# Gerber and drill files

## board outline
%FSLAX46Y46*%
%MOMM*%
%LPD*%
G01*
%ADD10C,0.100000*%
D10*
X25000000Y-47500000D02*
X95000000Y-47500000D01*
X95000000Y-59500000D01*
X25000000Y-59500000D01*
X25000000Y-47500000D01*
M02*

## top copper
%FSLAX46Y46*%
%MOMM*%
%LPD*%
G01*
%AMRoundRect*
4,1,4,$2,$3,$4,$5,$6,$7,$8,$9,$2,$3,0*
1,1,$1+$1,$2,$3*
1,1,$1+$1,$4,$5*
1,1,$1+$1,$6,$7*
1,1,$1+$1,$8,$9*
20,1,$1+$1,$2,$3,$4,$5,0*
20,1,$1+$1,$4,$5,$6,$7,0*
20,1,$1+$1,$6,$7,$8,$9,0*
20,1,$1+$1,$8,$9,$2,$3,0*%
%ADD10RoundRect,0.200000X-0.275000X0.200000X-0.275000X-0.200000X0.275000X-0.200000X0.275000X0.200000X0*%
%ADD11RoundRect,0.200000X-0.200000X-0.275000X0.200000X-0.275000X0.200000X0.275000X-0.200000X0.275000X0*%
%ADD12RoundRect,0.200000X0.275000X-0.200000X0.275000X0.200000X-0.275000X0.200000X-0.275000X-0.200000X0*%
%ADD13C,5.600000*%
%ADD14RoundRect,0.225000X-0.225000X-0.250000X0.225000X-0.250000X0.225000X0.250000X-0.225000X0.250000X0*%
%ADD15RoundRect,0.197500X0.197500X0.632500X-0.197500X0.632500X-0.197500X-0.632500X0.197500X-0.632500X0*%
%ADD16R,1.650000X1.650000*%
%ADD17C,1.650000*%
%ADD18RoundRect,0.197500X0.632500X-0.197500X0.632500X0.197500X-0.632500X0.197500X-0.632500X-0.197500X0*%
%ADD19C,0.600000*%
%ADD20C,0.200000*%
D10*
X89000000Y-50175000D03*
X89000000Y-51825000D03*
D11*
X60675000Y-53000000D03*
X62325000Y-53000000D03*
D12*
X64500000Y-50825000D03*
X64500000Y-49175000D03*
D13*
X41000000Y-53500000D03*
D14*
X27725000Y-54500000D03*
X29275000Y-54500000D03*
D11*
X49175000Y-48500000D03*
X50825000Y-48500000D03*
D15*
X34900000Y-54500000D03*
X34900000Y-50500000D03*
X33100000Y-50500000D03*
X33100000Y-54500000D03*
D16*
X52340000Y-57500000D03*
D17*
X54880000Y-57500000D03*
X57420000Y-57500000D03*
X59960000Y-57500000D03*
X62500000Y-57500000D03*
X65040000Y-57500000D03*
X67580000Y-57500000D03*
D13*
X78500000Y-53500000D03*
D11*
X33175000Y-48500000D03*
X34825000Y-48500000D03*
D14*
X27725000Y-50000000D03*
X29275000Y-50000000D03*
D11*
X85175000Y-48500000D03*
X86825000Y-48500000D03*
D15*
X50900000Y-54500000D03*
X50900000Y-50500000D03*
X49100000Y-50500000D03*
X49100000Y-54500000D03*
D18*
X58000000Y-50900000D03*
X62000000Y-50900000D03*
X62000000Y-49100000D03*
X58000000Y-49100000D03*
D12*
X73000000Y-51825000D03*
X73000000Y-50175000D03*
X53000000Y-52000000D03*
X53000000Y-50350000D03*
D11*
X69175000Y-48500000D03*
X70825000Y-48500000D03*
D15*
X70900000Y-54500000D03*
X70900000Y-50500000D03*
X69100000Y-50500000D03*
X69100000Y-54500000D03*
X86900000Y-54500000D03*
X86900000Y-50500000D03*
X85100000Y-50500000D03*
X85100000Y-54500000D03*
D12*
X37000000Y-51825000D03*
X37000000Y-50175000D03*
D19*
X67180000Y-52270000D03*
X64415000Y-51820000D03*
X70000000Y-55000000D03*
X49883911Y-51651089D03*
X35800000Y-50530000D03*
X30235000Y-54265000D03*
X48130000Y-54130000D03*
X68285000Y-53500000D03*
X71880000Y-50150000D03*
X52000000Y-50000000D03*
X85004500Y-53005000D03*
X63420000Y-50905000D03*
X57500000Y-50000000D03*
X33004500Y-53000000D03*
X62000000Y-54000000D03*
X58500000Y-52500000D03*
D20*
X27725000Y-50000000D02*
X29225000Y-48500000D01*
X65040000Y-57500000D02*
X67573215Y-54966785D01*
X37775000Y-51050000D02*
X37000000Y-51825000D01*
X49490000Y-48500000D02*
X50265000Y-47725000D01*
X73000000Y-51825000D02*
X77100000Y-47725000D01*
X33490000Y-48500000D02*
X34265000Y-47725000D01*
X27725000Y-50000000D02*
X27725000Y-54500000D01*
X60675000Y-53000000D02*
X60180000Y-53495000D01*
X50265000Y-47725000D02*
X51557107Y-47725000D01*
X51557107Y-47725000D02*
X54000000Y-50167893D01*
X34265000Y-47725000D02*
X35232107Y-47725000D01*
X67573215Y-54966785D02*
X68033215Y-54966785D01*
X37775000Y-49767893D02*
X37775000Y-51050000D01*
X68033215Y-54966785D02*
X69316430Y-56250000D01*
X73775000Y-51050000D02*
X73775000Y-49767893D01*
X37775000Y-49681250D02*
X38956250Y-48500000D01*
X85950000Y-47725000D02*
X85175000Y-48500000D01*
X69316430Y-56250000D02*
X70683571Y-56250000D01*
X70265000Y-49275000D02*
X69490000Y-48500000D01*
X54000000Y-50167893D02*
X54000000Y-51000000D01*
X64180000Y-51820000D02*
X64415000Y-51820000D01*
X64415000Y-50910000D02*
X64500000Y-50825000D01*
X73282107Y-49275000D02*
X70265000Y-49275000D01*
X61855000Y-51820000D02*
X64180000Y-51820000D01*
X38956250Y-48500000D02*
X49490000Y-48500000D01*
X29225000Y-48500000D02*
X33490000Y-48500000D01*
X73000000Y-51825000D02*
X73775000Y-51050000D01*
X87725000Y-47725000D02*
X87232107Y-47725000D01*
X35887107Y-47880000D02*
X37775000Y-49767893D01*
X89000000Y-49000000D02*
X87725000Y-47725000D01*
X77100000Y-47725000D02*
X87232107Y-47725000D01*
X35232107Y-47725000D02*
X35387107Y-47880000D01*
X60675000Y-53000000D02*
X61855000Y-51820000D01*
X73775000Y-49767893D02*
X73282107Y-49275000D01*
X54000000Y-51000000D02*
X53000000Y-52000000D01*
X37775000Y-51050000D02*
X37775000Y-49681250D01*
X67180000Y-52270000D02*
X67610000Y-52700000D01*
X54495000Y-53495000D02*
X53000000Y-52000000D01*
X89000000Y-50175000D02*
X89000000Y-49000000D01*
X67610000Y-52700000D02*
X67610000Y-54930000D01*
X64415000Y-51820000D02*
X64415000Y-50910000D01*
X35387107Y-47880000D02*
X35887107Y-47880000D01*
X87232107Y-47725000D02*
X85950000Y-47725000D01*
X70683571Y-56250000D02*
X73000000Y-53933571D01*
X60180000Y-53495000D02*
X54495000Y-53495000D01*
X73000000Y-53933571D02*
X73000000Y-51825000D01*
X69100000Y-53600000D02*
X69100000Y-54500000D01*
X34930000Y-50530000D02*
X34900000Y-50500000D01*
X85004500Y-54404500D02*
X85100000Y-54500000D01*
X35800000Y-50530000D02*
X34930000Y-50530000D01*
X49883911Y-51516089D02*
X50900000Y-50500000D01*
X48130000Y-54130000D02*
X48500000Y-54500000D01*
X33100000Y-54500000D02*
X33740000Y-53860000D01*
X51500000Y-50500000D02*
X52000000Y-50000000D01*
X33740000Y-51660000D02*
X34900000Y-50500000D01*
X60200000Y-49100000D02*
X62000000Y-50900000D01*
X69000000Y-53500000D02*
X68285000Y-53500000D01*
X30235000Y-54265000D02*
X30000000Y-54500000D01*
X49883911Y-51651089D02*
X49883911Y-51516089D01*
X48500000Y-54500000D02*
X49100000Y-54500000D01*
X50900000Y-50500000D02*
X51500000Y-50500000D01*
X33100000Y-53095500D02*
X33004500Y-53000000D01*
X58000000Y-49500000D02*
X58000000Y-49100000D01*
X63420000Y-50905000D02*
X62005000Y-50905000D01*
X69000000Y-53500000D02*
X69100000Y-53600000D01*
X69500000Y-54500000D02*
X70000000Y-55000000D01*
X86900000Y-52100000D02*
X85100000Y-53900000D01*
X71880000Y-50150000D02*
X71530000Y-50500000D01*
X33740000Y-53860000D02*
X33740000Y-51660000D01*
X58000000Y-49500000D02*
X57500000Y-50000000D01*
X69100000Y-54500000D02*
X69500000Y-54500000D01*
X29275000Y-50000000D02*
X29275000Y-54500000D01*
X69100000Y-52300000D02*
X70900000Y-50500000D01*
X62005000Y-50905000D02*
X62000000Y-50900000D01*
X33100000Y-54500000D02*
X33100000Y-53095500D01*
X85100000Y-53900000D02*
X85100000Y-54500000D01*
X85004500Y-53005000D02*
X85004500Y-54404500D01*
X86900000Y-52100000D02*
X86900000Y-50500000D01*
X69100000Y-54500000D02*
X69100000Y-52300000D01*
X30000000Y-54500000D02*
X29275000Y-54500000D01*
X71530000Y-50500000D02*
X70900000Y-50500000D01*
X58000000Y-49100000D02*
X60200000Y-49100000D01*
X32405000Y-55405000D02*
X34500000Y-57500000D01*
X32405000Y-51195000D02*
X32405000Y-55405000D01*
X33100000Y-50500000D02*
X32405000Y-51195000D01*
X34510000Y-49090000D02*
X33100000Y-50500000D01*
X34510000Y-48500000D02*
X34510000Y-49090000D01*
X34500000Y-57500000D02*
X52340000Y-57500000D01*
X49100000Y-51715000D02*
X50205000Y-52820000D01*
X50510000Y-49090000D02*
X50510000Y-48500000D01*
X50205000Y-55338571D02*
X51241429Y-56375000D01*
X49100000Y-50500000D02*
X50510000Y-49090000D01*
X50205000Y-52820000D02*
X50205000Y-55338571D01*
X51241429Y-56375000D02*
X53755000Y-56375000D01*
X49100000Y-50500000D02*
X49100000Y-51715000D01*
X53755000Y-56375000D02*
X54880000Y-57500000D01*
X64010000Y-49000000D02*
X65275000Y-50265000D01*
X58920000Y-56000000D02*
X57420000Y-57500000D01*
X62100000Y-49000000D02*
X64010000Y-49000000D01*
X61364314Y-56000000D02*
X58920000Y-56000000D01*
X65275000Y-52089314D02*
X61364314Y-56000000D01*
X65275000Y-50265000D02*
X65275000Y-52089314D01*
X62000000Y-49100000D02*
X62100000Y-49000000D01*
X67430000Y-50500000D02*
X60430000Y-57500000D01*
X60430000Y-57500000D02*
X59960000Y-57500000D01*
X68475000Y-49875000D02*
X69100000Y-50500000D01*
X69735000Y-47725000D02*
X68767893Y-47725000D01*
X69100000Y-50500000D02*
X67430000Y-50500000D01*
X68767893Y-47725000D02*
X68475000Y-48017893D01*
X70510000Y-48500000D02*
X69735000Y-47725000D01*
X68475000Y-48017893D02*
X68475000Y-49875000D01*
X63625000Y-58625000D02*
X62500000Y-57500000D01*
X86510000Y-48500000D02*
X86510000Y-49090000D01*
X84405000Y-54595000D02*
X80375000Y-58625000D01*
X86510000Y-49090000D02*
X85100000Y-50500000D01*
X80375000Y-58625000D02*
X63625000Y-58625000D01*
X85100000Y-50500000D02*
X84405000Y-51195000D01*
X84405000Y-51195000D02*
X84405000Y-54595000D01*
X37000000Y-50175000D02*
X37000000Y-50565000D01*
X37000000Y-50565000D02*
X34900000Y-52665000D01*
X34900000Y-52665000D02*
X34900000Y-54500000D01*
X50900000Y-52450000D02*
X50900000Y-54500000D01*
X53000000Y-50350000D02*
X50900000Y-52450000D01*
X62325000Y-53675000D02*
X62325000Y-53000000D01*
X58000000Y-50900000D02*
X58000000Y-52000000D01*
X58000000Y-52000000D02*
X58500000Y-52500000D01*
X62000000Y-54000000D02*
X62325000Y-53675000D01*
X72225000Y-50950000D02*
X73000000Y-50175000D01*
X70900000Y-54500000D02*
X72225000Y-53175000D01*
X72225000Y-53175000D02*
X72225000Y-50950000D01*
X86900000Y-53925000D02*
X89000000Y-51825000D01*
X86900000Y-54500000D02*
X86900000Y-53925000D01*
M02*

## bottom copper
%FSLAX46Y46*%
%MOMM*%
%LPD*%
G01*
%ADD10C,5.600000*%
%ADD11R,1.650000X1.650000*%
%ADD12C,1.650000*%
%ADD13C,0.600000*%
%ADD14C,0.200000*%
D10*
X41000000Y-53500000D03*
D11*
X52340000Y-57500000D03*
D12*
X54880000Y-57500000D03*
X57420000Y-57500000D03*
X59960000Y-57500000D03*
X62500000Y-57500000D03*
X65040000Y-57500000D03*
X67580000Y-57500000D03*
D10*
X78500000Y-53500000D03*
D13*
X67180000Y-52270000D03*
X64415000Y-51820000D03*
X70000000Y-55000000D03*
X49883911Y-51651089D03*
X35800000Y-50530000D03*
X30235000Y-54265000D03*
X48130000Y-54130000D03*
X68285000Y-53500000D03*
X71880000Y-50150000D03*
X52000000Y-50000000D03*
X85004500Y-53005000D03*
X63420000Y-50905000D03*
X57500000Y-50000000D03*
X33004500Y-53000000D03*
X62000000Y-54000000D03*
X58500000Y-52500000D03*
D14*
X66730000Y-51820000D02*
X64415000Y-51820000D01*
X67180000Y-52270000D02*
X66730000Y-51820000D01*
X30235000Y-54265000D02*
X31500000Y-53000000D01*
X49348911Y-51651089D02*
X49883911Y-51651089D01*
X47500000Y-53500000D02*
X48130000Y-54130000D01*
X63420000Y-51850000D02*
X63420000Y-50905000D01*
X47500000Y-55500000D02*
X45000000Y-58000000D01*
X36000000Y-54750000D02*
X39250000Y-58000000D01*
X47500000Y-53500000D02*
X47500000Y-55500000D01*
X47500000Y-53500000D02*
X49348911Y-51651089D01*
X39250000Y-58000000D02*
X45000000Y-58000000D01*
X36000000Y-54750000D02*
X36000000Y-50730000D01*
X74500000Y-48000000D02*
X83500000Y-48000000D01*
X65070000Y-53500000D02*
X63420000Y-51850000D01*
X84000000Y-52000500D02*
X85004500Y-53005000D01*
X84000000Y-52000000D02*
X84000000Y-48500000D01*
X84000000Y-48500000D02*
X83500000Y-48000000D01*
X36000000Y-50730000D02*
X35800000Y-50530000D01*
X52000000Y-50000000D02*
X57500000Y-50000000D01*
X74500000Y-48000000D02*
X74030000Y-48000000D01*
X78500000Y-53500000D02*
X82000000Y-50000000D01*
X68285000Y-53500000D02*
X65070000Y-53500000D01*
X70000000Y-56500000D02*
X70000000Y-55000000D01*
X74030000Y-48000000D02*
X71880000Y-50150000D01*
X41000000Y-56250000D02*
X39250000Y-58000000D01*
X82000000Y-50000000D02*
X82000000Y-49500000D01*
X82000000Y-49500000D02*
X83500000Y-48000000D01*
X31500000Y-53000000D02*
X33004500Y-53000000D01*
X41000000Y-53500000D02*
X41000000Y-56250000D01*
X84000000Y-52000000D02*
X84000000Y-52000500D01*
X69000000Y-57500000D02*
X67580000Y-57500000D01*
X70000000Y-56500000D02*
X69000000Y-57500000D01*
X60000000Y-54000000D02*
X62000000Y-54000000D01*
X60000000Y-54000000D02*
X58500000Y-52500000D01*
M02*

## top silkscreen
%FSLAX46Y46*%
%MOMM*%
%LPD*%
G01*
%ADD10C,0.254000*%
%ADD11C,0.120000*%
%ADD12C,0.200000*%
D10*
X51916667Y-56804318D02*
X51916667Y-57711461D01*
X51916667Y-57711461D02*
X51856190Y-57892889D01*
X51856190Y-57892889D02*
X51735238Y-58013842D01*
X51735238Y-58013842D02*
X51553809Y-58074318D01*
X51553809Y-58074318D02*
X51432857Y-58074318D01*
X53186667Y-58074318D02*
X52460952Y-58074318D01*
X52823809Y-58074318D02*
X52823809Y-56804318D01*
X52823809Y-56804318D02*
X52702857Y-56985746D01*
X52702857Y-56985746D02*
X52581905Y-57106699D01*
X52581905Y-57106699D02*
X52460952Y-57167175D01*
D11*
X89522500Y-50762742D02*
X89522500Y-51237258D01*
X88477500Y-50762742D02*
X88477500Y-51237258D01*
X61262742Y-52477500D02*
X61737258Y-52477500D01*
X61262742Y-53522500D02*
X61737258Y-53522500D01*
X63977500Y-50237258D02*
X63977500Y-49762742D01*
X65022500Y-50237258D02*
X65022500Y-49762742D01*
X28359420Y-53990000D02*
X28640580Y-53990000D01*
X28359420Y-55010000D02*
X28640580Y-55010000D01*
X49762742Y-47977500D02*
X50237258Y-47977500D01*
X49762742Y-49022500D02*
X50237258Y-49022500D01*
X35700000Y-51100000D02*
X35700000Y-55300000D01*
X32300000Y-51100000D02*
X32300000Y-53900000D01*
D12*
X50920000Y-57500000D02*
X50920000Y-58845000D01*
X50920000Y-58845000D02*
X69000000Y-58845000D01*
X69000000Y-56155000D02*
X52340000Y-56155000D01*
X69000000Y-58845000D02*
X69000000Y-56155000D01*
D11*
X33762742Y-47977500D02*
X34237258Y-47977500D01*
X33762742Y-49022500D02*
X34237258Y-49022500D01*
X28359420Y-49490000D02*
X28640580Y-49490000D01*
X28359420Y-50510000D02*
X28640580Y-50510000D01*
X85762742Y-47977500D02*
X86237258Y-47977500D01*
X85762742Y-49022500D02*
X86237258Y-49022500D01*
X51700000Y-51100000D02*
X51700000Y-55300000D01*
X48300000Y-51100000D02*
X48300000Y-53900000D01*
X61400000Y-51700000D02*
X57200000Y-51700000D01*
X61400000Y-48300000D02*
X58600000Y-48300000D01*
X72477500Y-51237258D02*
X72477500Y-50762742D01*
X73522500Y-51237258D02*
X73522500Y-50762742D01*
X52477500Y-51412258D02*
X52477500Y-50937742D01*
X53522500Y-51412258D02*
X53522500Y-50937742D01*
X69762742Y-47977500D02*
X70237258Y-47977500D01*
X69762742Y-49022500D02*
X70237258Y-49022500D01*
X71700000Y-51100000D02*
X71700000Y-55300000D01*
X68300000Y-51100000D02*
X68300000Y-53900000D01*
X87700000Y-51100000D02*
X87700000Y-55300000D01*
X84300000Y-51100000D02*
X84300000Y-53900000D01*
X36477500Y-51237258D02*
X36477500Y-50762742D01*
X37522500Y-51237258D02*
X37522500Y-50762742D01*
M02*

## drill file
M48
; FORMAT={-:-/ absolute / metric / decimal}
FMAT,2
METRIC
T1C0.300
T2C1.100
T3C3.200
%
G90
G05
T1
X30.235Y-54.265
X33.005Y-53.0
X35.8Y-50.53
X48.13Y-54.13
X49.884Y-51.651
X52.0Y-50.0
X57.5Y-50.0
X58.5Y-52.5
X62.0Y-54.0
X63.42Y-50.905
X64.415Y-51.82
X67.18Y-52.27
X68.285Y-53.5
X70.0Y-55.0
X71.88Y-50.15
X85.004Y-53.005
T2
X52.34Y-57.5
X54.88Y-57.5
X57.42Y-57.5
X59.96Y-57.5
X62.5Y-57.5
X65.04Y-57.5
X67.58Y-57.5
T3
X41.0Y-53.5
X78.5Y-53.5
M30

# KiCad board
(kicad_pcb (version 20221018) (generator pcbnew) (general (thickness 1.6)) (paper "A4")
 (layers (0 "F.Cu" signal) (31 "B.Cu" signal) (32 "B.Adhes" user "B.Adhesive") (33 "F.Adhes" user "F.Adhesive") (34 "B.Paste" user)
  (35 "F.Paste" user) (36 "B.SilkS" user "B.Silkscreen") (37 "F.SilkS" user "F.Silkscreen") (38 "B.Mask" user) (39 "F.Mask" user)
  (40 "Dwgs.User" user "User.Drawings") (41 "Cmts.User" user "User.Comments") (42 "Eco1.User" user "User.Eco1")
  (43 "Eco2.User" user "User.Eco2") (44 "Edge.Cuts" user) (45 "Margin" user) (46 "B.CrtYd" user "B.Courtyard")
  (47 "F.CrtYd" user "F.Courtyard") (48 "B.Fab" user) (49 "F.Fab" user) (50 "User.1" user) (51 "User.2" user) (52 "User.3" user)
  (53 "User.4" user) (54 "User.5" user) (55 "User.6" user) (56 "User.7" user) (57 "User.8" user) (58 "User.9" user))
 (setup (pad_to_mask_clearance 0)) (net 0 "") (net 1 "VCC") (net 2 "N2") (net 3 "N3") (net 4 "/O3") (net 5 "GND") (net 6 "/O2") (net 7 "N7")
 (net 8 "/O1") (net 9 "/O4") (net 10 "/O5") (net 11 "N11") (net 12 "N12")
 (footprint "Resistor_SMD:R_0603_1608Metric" (layer "F.Cu") (at 89 51 -90)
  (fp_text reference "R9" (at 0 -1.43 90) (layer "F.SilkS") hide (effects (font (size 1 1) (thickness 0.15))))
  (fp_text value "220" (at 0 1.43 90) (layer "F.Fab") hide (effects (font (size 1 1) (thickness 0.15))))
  (fp_line (start -0.237258 -0.5225) (end 0.237258 -0.5225) (stroke (width 0.12) (type solid)) (layer "F.SilkS"))
  (fp_line (start -0.237258 0.5225) (end 0.237258 0.5225) (stroke (width 0.12) (type solid)) (layer "F.SilkS"))
  (pad "1" smd roundrect (at -0.825 0 270) (size 0.8 0.95) (layers "F.Cu" "F.Paste" "F.Mask") (roundrect_rratio 0.25) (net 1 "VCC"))
  (pad "2" smd roundrect (at 0.825 0 270) (size 0.8 0.95) (layers "F.Cu" "F.Paste" "F.Mask") (roundrect_rratio 0.25) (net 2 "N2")))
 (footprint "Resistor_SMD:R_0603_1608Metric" (layer "F.Cu") (at 61.5 53)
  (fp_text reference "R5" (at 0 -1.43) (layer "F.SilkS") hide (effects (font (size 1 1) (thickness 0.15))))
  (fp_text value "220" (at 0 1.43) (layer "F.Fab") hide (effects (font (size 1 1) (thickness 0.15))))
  (fp_line (start -0.237258 -0.5225) (end 0.237258 -0.5225) (stroke (width 0.12) (type solid)) (layer "F.SilkS"))
  (fp_line (start -0.237258 0.5225) (end 0.237258 0.5225) (stroke (width 0.12) (type solid)) (layer "F.SilkS"))
  (pad "1" smd roundrect (at -0.825 0) (size 0.8 0.95) (layers "F.Cu" "F.Paste" "F.Mask") (roundrect_rratio 0.25) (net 1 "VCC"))
  (pad "2" smd roundrect (at 0.825 0) (size 0.8 0.95) (layers "F.Cu" "F.Paste" "F.Mask") (roundrect_rratio 0.25) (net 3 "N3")))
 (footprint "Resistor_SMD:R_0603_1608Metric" (layer "F.Cu") (at 64.5 50 90)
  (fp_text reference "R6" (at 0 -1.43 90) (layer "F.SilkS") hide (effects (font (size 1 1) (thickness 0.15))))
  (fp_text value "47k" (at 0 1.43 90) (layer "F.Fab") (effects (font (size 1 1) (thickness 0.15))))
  (fp_line (start -0.237258 -0.5225) (end 0.237258 -0.5225) (stroke (width 0.12) (type solid)) (layer "F.SilkS"))
  (fp_line (start -0.237258 0.5225) (end 0.237258 0.5225) (stroke (width 0.12) (type solid)) (layer "F.SilkS"))
  (pad "1" smd roundrect (at -0.825 0 90) (size 0.8 0.95) (layers "F.Cu" "F.Paste" "F.Mask") (roundrect_rratio 0.25) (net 1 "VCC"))
  (pad "2" smd roundrect (at 0.825 0 90) (size 0.8 0.95) (layers "F.Cu" "F.Paste" "F.Mask") (roundrect_rratio 0.25) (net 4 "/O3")))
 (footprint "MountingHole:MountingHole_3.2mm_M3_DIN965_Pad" (layer "F.Cu") (at 41 53.5)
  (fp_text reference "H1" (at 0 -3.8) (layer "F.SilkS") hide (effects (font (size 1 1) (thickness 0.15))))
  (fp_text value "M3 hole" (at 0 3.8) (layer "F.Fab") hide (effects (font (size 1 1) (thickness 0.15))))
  (pad "1" thru_hole circle (at 0 0) (size 5.6 5.6) (drill 3.2) (layers "*.Cu" "*.Mask") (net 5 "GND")))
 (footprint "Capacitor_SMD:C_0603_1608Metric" (layer "F.Cu") (at 28.5 54.5)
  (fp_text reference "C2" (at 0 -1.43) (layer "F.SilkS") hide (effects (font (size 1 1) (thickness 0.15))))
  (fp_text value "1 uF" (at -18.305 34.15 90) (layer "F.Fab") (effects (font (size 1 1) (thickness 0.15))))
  (fp_line (start -0.14058 -0.51) (end 0.14058 -0.51) (stroke (width 0.12) (type solid)) (layer "F.SilkS"))
  (fp_line (start -0.14058 0.51) (end 0.14058 0.51) (stroke (width 0.12) (type solid)) (layer "F.SilkS"))
  (pad "1" smd roundrect (at -0.775 0) (size 0.9 0.95) (layers "F.Cu" "F.Paste" "F.Mask") (roundrect_rratio 0.25) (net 1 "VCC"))
  (pad "2" smd roundrect (at 0.775 0) (size 0.9 0.95) (layers "F.Cu" "F.Paste" "F.Mask") (roundrect_rratio 0.25) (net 5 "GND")))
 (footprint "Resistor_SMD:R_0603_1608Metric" (layer "F.Cu") (at 50 48.5)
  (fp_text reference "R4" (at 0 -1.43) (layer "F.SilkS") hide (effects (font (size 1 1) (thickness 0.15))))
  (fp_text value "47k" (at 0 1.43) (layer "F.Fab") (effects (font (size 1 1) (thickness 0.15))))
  (fp_line (start -0.237258 -0.5225) (end 0.237258 -0.5225) (stroke (width 0.12) (type solid)) (layer "F.SilkS"))
  (fp_line (start -0.237258 0.5225) (end 0.237258 0.5225) (stroke (width 0.12) (type solid)) (layer "F.SilkS"))
  (pad "1" smd roundrect (at -0.825 0) (size 0.8 0.95) (layers "F.Cu" "F.Paste" "F.Mask") (roundrect_rratio 0.25) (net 1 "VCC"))
  (pad "2" smd roundrect (at 0.825 0) (size 0.8 0.95) (layers "F.Cu" "F.Paste" "F.Mask") (roundrect_rratio 0.25) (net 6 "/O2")))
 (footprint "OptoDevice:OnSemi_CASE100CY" (layer "F.Cu") (at 34 52.5 180)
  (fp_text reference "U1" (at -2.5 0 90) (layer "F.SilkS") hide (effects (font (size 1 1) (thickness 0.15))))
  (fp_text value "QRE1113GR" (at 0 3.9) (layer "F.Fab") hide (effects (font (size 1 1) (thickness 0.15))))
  (fp_line (start -1.7 1.4) (end -1.7 -2.8) (stroke (width 0.12) (type solid)) (layer "F.SilkS"))
  (fp_line (start 1.7 1.4) (end 1.7 -1.4) (stroke (width 0.12) (type solid)) (layer "F.SilkS"))
  (pad "1" smd roundrect (at -0.9 -2 180) (size 0.79 1.66) (layers "F.Cu" "F.Paste" "F.Mask") (roundrect_rratio 0.25) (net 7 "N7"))
  (pad "2" smd roundrect (at -0.9 2 180) (size 0.79 1.66) (layers "F.Cu" "F.Paste" "F.Mask") (roundrect_rratio 0.25) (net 5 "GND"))
  (pad "3" smd roundrect (at 0.9 2 180) (size 0.79 1.66) (layers "F.Cu" "F.Paste" "F.Mask") (roundrect_rratio 0.25) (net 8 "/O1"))
  (pad "4" smd roundrect (at 0.9 -2 180) (size 0.79 1.66) (layers "F.Cu" "F.Paste" "F.Mask") (roundrect_rratio 0.25) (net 5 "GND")))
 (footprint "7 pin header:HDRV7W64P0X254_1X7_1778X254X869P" (layer "F.Cu") (at 52.34 57.5)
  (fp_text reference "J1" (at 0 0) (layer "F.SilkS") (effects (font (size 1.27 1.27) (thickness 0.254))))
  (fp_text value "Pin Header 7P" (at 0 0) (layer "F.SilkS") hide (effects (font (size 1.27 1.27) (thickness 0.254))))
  (fp_line (start -1.42 0) (end -1.42 1.345) (stroke (width 0.2) (type solid)) (layer "F.SilkS"))
  (fp_line (start -1.42 1.345) (end 16.66 1.345) (stroke (width 0.2) (type solid)) (layer "F.SilkS"))
  (fp_line (start 16.66 -1.345) (end 0 -1.345) (stroke (width 0.2) (type solid)) (layer "F.SilkS"))
  (fp_line (start 16.66 1.345) (end 16.66 -1.345) (stroke (width 0.2) (type solid)) (layer "F.SilkS"))
  (pad "1" thru_hole rect (at 0 0) (size 1.65 1.65) (drill 1.1) (layers "*.Cu" "*.Mask") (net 8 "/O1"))
  (pad "2" thru_hole circle (at 2.54 0) (size 1.65 1.65) (drill 1.1) (layers "*.Cu" "*.Mask") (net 6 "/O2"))
  (pad "3" thru_hole circle (at 5.08 0) (size 1.65 1.65) (drill 1.1) (layers "*.Cu" "*.Mask") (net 4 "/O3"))
  (pad "4" thru_hole circle (at 7.62 0) (size 1.65 1.65) (drill 1.1) (layers "*.Cu" "*.Mask") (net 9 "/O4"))
  (pad "5" thru_hole circle (at 10.16 0) (size 1.65 1.65) (drill 1.1) (layers "*.Cu" "*.Mask") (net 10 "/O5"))
  (pad "6" thru_hole circle (at 12.7 0) (size 1.65 1.65) (drill 1.1) (layers "*.Cu" "*.Mask") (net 1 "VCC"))
  (pad "7" thru_hole circle (at 15.24 0) (size 1.65 1.65) (drill 1.1) (layers "*.Cu" "*.Mask") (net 5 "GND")))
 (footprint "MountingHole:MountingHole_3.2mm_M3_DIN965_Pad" (layer "F.Cu") (at 78.5 53.5)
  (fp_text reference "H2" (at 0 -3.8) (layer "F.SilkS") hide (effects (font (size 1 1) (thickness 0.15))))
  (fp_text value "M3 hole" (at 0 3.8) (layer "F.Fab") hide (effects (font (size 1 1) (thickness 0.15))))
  (pad "1" thru_hole circle (at 0 0) (size 5.6 5.6) (drill 3.2) (layers "*.Cu" "*.Mask") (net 5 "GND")))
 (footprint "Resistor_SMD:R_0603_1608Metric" (layer "F.Cu") (at 34 48.5)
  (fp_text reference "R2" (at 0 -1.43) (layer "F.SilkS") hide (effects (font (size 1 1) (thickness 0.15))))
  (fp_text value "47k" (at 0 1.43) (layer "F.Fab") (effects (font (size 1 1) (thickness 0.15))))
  (fp_line (start -0.237258 -0.5225) (end 0.237258 -0.5225) (stroke (width 0.12) (type solid)) (layer "F.SilkS"))
  (fp_line (start -0.237258 0.5225) (end 0.237258 0.5225) (stroke (width 0.12) (type solid)) (layer "F.SilkS"))
  (pad "1" smd roundrect (at -0.825 0) (size 0.8 0.95) (layers "F.Cu" "F.Paste" "F.Mask") (roundrect_rratio 0.25) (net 1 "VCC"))
  (pad "2" smd roundrect (at 0.825 0) (size 0.8 0.95) (layers "F.Cu" "F.Paste" "F.Mask") (roundrect_rratio 0.25) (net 8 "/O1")))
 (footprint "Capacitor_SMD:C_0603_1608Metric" (layer "F.Cu") (at 28.5 50)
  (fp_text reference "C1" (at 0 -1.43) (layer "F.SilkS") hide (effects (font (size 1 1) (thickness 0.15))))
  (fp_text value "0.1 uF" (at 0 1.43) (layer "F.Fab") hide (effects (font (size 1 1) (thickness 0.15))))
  (fp_line (start -0.14058 -0.51) (end 0.14058 -0.51) (stroke (width 0.12) (type solid)) (layer "F.SilkS"))
  (fp_line (start -0.14058 0.51) (end 0.14058 0.51) (stroke (width 0.12) (type solid)) (layer "F.SilkS"))
  (pad "1" smd roundrect (at -0.775 0) (size 0.9 0.95) (layers "F.Cu" "F.Paste" "F.Mask") (roundrect_rratio 0.25) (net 1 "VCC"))
  (pad "2" smd roundrect (at 0.775 0) (size 0.9 0.95) (layers "F.Cu" "F.Paste" "F.Mask") (roundrect_rratio 0.25) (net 5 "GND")))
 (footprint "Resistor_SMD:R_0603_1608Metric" (layer "F.Cu") (at 86 48.5)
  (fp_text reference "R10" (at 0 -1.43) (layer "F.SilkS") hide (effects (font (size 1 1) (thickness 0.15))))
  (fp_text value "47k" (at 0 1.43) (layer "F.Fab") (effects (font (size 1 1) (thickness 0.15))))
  (fp_line (start -0.237258 -0.5225) (end 0.237258 -0.5225) (stroke (width 0.12) (type solid)) (layer "F.SilkS"))
  (fp_line (start -0.237258 0.5225) (end 0.237258 0.5225) (stroke (width 0.12) (type solid)) (layer "F.SilkS"))
  (pad "1" smd roundrect (at -0.825 0) (size 0.8 0.95) (layers "F.Cu" "F.Paste" "F.Mask") (roundrect_rratio 0.25) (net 1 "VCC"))
  (pad "2" smd roundrect (at 0.825 0) (size 0.8 0.95) (layers "F.Cu" "F.Paste" "F.Mask") (roundrect_rratio 0.25) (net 10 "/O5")))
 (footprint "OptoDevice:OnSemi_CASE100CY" (layer "F.Cu") (at 50 52.5 180)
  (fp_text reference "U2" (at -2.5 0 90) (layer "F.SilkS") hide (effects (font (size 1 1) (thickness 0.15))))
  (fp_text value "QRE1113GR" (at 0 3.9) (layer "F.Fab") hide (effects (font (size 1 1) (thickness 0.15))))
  (fp_line (start -1.7 1.4) (end -1.7 -2.8) (stroke (width 0.12) (type solid)) (layer "F.SilkS"))
  (fp_line (start 1.7 1.4) (end 1.7 -1.4) (stroke (width 0.12) (type solid)) (layer "F.SilkS"))
  (pad "1" smd roundrect (at -0.9 -2 180) (size 0.79 1.66) (layers "F.Cu" "F.Paste" "F.Mask") (roundrect_rratio 0.25) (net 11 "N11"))
  (pad "2" smd roundrect (at -0.9 2 180) (size 0.79 1.66) (layers "F.Cu" "F.Paste" "F.Mask") (roundrect_rratio 0.25) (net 5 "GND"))
  (pad "3" smd roundrect (at 0.9 2 180) (size 0.79 1.66) (layers "F.Cu" "F.Paste" "F.Mask") (roundrect_rratio 0.25) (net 6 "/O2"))
  (pad "4" smd roundrect (at 0.9 -2 180) (size 0.79 1.66) (layers "F.Cu" "F.Paste" "F.Mask") (roundrect_rratio 0.25) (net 5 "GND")))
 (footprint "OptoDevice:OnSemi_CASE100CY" (layer "F.Cu") (at 60 50 90)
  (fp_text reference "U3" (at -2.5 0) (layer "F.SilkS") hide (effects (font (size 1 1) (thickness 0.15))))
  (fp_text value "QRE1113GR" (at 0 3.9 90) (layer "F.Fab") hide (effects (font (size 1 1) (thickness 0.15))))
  (fp_line (start -1.7 1.4) (end -1.7 -2.8) (stroke (width 0.12) (type solid)) (layer "F.SilkS"))
  (fp_line (start 1.7 1.4) (end 1.7 -1.4) (stroke (width 0.12) (type solid)) (layer "F.SilkS"))
  (pad "1" smd roundrect (at -0.9 -2 90) (size 0.79 1.66) (layers "F.Cu" "F.Paste" "F.Mask") (roundrect_rratio 0.25) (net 3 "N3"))
  (pad "2" smd roundrect (at -0.9 2 90) (size 0.79 1.66) (layers "F.Cu" "F.Paste" "F.Mask") (roundrect_rratio 0.25) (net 5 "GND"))
  (pad "3" smd roundrect (at 0.9 2 90) (size 0.79 1.66) (layers "F.Cu" "F.Paste" "F.Mask") (roundrect_rratio 0.25) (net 4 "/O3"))
  (pad "4" smd roundrect (at 0.9 -2 90) (size 0.79 1.66) (layers "F.Cu" "F.Paste" "F.Mask") (roundrect_rratio 0.25) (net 5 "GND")))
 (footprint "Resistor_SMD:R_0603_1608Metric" (layer "F.Cu") (at 73 51 90)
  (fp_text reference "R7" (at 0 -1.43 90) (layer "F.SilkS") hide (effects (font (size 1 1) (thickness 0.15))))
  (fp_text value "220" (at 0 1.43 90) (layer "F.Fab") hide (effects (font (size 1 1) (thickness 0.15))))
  (fp_line (start -0.237258 -0.5225) (end 0.237258 -0.5225) (stroke (width 0.12) (type solid)) (layer "F.SilkS"))
  (fp_line (start -0.237258 0.5225) (end 0.237258 0.5225) (stroke (width 0.12) (type solid)) (layer "F.SilkS"))
  (pad "1" smd roundrect (at -0.825 0 90) (size 0.8 0.95) (layers "F.Cu" "F.Paste" "F.Mask") (roundrect_rratio 0.25) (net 1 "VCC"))
  (pad "2" smd roundrect (at 0.825 0 90) (size 0.8 0.95) (layers "F.Cu" "F.Paste" "F.Mask") (roundrect_rratio 0.25) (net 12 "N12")))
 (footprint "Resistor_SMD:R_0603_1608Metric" (layer "F.Cu") (at 53 51.175 90)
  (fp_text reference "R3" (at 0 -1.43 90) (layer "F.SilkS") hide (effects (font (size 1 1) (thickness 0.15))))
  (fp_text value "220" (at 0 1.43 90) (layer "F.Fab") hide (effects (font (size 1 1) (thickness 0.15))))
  (fp_line (start -0.237258 -0.5225) (end 0.237258 -0.5225) (stroke (width 0.12) (type solid)) (layer "F.SilkS"))
  (fp_line (start -0.237258 0.5225) (end 0.237258 0.5225) (stroke (width 0.12) (type solid)) (layer "F.SilkS"))
  (pad "1" smd roundrect (at -0.825 0 90) (size 0.8 0.95) (layers "F.Cu" "F.Paste" "F.Mask") (roundrect_rratio 0.25) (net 1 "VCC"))
  (pad "2" smd roundrect (at 0.825 0 90) (size 0.8 0.95) (layers "F.Cu" "F.Paste" "F.Mask") (roundrect_rratio 0.25) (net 11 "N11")))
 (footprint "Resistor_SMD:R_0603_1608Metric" (layer "F.Cu") (at 70 48.5)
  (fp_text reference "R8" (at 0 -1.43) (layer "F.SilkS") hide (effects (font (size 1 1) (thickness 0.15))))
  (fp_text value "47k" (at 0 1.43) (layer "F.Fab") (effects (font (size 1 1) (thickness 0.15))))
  (fp_line (start -0.237258 -0.5225) (end 0.237258 -0.5225) (stroke (width 0.12) (type solid)) (layer "F.SilkS"))
  (fp_line (start -0.237258 0.5225) (end 0.237258 0.5225) (stroke (width 0.12) (type solid)) (layer "F.SilkS"))
  (pad "1" smd roundrect (at -0.825 0) (size 0.8 0.95) (layers "F.Cu" "F.Paste" "F.Mask") (roundrect_rratio 0.25) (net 1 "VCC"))
  (pad "2" smd roundrect (at 0.825 0) (size 0.8 0.95) (layers "F.Cu" "F.Paste" "F.Mask") (roundrect_rratio 0.25) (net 9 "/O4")))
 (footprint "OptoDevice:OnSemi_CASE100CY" (layer "F.Cu") (at 70 52.5 180)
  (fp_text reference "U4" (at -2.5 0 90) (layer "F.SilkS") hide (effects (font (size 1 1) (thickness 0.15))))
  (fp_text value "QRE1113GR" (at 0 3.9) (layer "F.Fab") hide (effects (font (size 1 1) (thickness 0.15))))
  (fp_line (start -1.7 1.4) (end -1.7 -2.8) (stroke (width 0.12) (type solid)) (layer "F.SilkS"))
  (fp_line (start 1.7 1.4) (end 1.7 -1.4) (stroke (width 0.12) (type solid)) (layer "F.SilkS"))
  (pad "1" smd roundrect (at -0.9 -2 180) (size 0.79 1.66) (layers "F.Cu" "F.Paste" "F.Mask") (roundrect_rratio 0.25) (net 12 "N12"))
  (pad "2" smd roundrect (at -0.9 2 180) (size 0.79 1.66) (layers "F.Cu" "F.Paste" "F.Mask") (roundrect_rratio 0.25) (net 5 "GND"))
  (pad "3" smd roundrect (at 0.9 2 180) (size 0.79 1.66) (layers "F.Cu" "F.Paste" "F.Mask") (roundrect_rratio 0.25) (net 9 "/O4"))
  (pad "4" smd roundrect (at 0.9 -2 180) (size 0.79 1.66) (layers "F.Cu" "F.Paste" "F.Mask") (roundrect_rratio 0.25) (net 5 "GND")))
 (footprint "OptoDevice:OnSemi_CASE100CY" (layer "F.Cu") (at 86 52.5 180)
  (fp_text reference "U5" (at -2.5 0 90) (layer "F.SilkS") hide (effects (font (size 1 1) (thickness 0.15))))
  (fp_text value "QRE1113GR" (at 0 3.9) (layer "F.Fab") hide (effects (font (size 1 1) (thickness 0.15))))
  (fp_line (start -1.7 1.4) (end -1.7 -2.8) (stroke (width 0.12) (type solid)) (layer "F.SilkS"))
  (fp_line (start 1.7 1.4) (end 1.7 -1.4) (stroke (width 0.12) (type solid)) (layer "F.SilkS"))
  (pad "1" smd roundrect (at -0.9 -2 180) (size 0.79 1.66) (layers "F.Cu" "F.Paste" "F.Mask") (roundrect_rratio 0.25) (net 2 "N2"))
  (pad "2" smd roundrect (at -0.9 2 180) (size 0.79 1.66) (layers "F.Cu" "F.Paste" "F.Mask") (roundrect_rratio 0.25) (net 5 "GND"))
  (pad "3" smd roundrect (at 0.9 2 180) (size 0.79 1.66) (layers "F.Cu" "F.Paste" "F.Mask") (roundrect_rratio 0.25) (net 10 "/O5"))
  (pad "4" smd roundrect (at 0.9 -2 180) (size 0.79 1.66) (layers "F.Cu" "F.Paste" "F.Mask") (roundrect_rratio 0.25) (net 5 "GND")))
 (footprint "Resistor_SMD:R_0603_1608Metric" (layer "F.Cu") (at 37 51 90)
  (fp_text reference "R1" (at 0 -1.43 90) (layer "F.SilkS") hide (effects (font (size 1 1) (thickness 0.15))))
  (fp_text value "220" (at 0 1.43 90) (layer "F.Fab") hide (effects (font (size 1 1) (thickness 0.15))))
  (fp_line (start -0.237258 -0.5225) (end 0.237258 -0.5225) (stroke (width 0.12) (type solid)) (layer "F.SilkS"))
  (fp_line (start -0.237258 0.5225) (end 0.237258 0.5225) (stroke (width 0.12) (type solid)) (layer "F.SilkS"))
  (pad "1" smd roundrect (at -0.825 0 90) (size 0.8 0.95) (layers "F.Cu" "F.Paste" "F.Mask") (roundrect_rratio 0.25) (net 1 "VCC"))
  (pad "2" smd roundrect (at 0.825 0 90) (size 0.8 0.95) (layers "F.Cu" "F.Paste" "F.Mask") (roundrect_rratio 0.25) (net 7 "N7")))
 (gr_rect (start 25 47.5) (end 95 59.5) (stroke (width 0.1) (type default)) (fill none) (layer "Edge.Cuts"))
 (segment (start 27.725 50) (end 29.225 48.5) (width 0.2) (layer "F.Cu") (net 1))
 (segment (start 65.04 57.5) (end 67.573215 54.966785) (width 0.2) (layer "F.Cu") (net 1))
 (segment (start 37.775 51.05) (end 37 51.825) (width 0.2) (layer "F.Cu") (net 1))
 (segment (start 49.49 48.5) (end 50.265 47.725) (width 0.2) (layer "F.Cu") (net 1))
 (segment (start 73 51.825) (end 77.1 47.725) (width 0.2) (layer "F.Cu") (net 1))
 (segment (start 33.49 48.5) (end 34.265 47.725) (width 0.2) (layer "F.Cu") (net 1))
 (segment (start 27.725 50) (end 27.725 54.5) (width 0.2) (layer "F.Cu") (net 1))
 (segment (start 60.675 53) (end 60.18 53.495) (width 0.2) (layer "F.Cu") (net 1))
 (segment (start 50.265 47.725) (end 51.557107 47.725) (width 0.2) (layer "F.Cu") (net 1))
 (segment (start 51.557107 47.725) (end 54 50.167893) (width 0.2) (layer "F.Cu") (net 1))
 (segment (start 34.265 47.725) (end 35.232107 47.725) (width 0.2) (layer "F.Cu") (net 1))
 (segment (start 67.573215 54.966785) (end 68.033215 54.966785) (width 0.2) (layer "F.Cu") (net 1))
 (segment (start 37.775 49.767893) (end 37.775 51.05) (width 0.2) (layer "F.Cu") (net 1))
 (segment (start 68.033215 54.966785) (end 69.31643 56.25) (width 0.2) (layer "F.Cu") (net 1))
 (segment (start 73.775 51.05) (end 73.775 49.767893) (width 0.2) (layer "F.Cu") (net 1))
 (segment (start 37.775 49.68125) (end 38.95625 48.5) (width 0.2) (layer "F.Cu") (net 1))
 (segment (start 85.95 47.725) (end 85.175 48.5) (width 0.2) (layer "F.Cu") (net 1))
 (segment (start 69.31643 56.25) (end 70.683571 56.25) (width 0.2) (layer "F.Cu") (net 1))
 (segment (start 70.265 49.275) (end 69.49 48.5) (width 0.2) (layer "F.Cu") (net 1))
 (segment (start 54 50.167893) (end 54 51) (width 0.2) (layer "F.Cu") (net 1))
 (segment (start 64.18 51.82) (end 64.415 51.82) (width 0.2) (layer "F.Cu") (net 1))
 (segment (start 64.415 50.91) (end 64.5 50.825) (width 0.2) (layer "F.Cu") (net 1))
 (segment (start 73.282107 49.275) (end 70.265 49.275) (width 0.2) (layer "F.Cu") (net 1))
 (segment (start 61.855 51.82) (end 64.18 51.82) (width 0.2) (layer "F.Cu") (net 1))
 (segment (start 38.95625 48.5) (end 49.49 48.5) (width 0.2) (layer "F.Cu") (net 1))
 (segment (start 29.225 48.5) (end 33.49 48.5) (width 0.2) (layer "F.Cu") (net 1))
 (segment (start 73 51.825) (end 73.775 51.05) (width 0.2) (layer "F.Cu") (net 1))
 (segment (start 87.725 47.725) (end 87.232107 47.725) (width 0.2) (layer "F.Cu") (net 1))
 (segment (start 35.887107 47.88) (end 37.775 49.767893) (width 0.2) (layer "F.Cu") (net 1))
 (segment (start 89 49) (end 87.725 47.725) (width 0.2) (layer "F.Cu") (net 1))
 (segment (start 77.1 47.725) (end 87.232107 47.725) (width 0.2) (layer "F.Cu") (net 1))
 (segment (start 35.232107 47.725) (end 35.387107 47.88) (width 0.2) (layer "F.Cu") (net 1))
 (segment (start 60.675 53) (end 61.855 51.82) (width 0.2) (layer "F.Cu") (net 1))
 (segment (start 73.775 49.767893) (end 73.282107 49.275) (width 0.2) (layer "F.Cu") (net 1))
 (segment (start 54 51) (end 53 52) (width 0.2) (layer "F.Cu") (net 1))
 (segment (start 37.775 51.05) (end 37.775 49.68125) (width 0.2) (layer "F.Cu") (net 1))
 (segment (start 67.18 52.27) (end 67.61 52.7) (width 0.2) (layer "F.Cu") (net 1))
 (segment (start 54.495 53.495) (end 53 52) (width 0.2) (layer "F.Cu") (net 1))
 (segment (start 89 50.175) (end 89 49) (width 0.2) (layer "F.Cu") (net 1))
 (segment (start 67.61 52.7) (end 67.61 54.93) (width 0.2) (layer "F.Cu") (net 1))
 (segment (start 64.415 51.82) (end 64.415 50.91) (width 0.2) (layer "F.Cu") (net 1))
 (segment (start 35.387107 47.88) (end 35.887107 47.88) (width 0.2) (layer "F.Cu") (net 1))
 (segment (start 87.232107 47.725) (end 85.95 47.725) (width 0.2) (layer "F.Cu") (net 1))
 (segment (start 70.683571 56.25) (end 73 53.933571) (width 0.2) (layer "F.Cu") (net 1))
 (segment (start 60.18 53.495) (end 54.495 53.495) (width 0.2) (layer "F.Cu") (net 1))
 (segment (start 73 53.933571) (end 73 51.825) (width 0.2) (layer "F.Cu") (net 1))
 (via (at 67.18 52.27) (size 0.6) (drill 0.3) (layers "F.Cu" "B.Cu") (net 1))
 (via (at 64.415 51.82) (size 0.6) (drill 0.3) (layers "F.Cu" "B.Cu") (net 1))
 (segment (start 66.73 51.82) (end 64.415 51.82) (width 0.2) (layer "B.Cu") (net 1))
 (segment (start 67.18 52.27) (end 66.73 51.82) (width 0.2) (layer "B.Cu") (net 1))
 (segment (start 69.1 53.6) (end 69.1 54.5) (width 0.2) (layer "F.Cu") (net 5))
 (segment (start 34.93 50.53) (end 34.9 50.5) (width 0.2) (layer "F.Cu") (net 5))
 (segment (start 85.0045 54.4045) (end 85.1 54.5) (width 0.2) (layer "F.Cu") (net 5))
 (segment (start 35.8 50.53) (end 34.93 50.53) (width 0.2) (layer "F.Cu") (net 5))
 (segment (start 49.883911 51.516089) (end 50.9 50.5) (width 0.2) (layer "F.Cu") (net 5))
 (segment (start 48.13 54.13) (end 48.5 54.5) (width 0.2) (layer "F.Cu") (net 5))
 (segment (start 33.1 54.5) (end 33.74 53.86) (width 0.2) (layer "F.Cu") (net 5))
 (segment (start 51.5 50.5) (end 52 50) (width 0.2) (layer "F.Cu") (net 5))
 (segment (start 33.74 51.66) (end 34.9 50.5) (width 0.2) (layer "F.Cu") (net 5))
 (segment (start 60.2 49.1) (end 62 50.9) (width 0.2) (layer "F.Cu") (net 5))
 (segment (start 69 53.5) (end 68.285 53.5) (width 0.2) (layer "F.Cu") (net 5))
 (segment (start 30.235 54.265) (end 30 54.5) (width 0.2) (layer "F.Cu") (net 5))
 (segment (start 49.883911 51.651089) (end 49.883911 51.516089) (width 0.2) (layer "F.Cu") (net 5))
 (segment (start 48.5 54.5) (end 49.1 54.5) (width 0.2) (layer "F.Cu") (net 5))
 (segment (start 50.9 50.5) (end 51.5 50.5) (width 0.2) (layer "F.Cu") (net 5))
 (segment (start 33.1 53.0955) (end 33.0045 53) (width 0.2) (layer "F.Cu") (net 5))
 (segment (start 58 49.5) (end 58 49.1) (width 0.2) (layer "F.Cu") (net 5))
 (segment (start 63.42 50.905) (end 62.005 50.905) (width 0.2) (layer "F.Cu") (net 5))
 (segment (start 69 53.5) (end 69.1 53.6) (width 0.2) (layer "F.Cu") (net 5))
 (segment (start 69.5 54.5) (end 70 55) (width 0.2) (layer "F.Cu") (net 5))
 (segment (start 86.9 52.1) (end 85.1 53.9) (width 0.2) (layer "F.Cu") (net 5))
 (segment (start 71.88 50.15) (end 71.53 50.5) (width 0.2) (layer "F.Cu") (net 5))
 (segment (start 33.74 53.86) (end 33.74 51.66) (width 0.2) (layer "F.Cu") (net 5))
 (segment (start 58 49.5) (end 57.5 50) (width 0.2) (layer "F.Cu") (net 5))
 (segment (start 69.1 54.5) (end 69.5 54.5) (width 0.2) (layer "F.Cu") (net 5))
 (segment (start 29.275 50) (end 29.275 54.5) (width 0.2) (layer "F.Cu") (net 5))
 (segment (start 69.1 52.3) (end 70.9 50.5) (width 0.2) (layer "F.Cu") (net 5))
 (segment (start 62.005 50.905) (end 62 50.9) (width 0.2) (layer "F.Cu") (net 5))
 (segment (start 33.1 54.5) (end 33.1 53.0955) (width 0.2) (layer "F.Cu") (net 5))
 (segment (start 85.1 53.9) (end 85.1 54.5) (width 0.2) (layer "F.Cu") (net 5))
 (segment (start 85.0045 53.005) (end 85.0045 54.4045) (width 0.2) (layer "F.Cu") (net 5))
 (segment (start 86.9 52.1) (end 86.9 50.5) (width 0.2) (layer "F.Cu") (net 5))
 (segment (start 69.1 54.5) (end 69.1 52.3) (width 0.2) (layer "F.Cu") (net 5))
 (segment (start 30 54.5) (end 29.275 54.5) (width 0.2) (layer "F.Cu") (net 5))
 (segment (start 71.53 50.5) (end 70.9 50.5) (width 0.2) (layer "F.Cu") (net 5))
 (segment (start 58 49.1) (end 60.2 49.1) (width 0.2) (layer "F.Cu") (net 5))
 (via (at 70 55) (size 0.6) (drill 0.3) (layers "F.Cu" "B.Cu") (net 5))
 (via (at 49.883911 51.651089) (size 0.6) (drill 0.3) (layers "F.Cu" "B.Cu") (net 5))
 (via (at 35.8 50.53) (size 0.6) (drill 0.3) (layers "F.Cu" "B.Cu") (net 5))
 (via (at 30.235 54.265) (size 0.6) (drill 0.3) (layers "F.Cu" "B.Cu") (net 5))
 (via (at 48.13 54.13) (size 0.6) (drill 0.3) (layers "F.Cu" "B.Cu") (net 5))
 (via (at 68.285 53.5) (size 0.6) (drill 0.3) (layers "F.Cu" "B.Cu") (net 5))
 (via (at 71.88 50.15) (size 0.6) (drill 0.3) (layers "F.Cu" "B.Cu") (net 5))
 (via (at 52 50) (size 0.6) (drill 0.3) (layers "F.Cu" "B.Cu") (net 5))
 (via (at 85.0045 53.005) (size 0.6) (drill 0.3) (layers "F.Cu" "B.Cu") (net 5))
 (via (at 63.42 50.905) (size 0.6) (drill 0.3) (layers "F.Cu" "B.Cu") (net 5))
 (via (at 57.5 50) (size 0.6) (drill 0.3) (layers "F.Cu" "B.Cu") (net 5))
 (via (at 33.0045 53) (size 0.6) (drill 0.3) (layers "F.Cu" "B.Cu") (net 5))
 (segment (start 30.235 54.265) (end 31.5 53) (width 0.2) (layer "B.Cu") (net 5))
 (segment (start 49.348911 51.651089) (end 49.883911 51.651089) (width 0.2) (layer "B.Cu") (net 5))
 (segment (start 47.5 53.5) (end 48.13 54.13) (width 0.2) (layer "B.Cu") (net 5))
 (segment (start 63.42 51.85) (end 63.42 50.905) (width 0.2) (layer "B.Cu") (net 5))
 (segment (start 47.5 55.5) (end 45 58) (width 0.2) (layer "B.Cu") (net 5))
 (segment (start 36 54.75) (end 39.25 58) (width 0.2) (layer "B.Cu") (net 5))
 (segment (start 47.5 53.5) (end 47.5 55.5) (width 0.2) (layer "B.Cu") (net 5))
 (segment (start 47.5 53.5) (end 49.348911 51.651089) (width 0.2) (layer "B.Cu") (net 5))
 (segment (start 39.25 58) (end 45 58) (width 0.2) (layer "B.Cu") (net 5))
 (segment (start 36 54.75) (end 36 50.73) (width 0.2) (layer "B.Cu") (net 5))
 (segment (start 74.5 48) (end 83.5 48) (width 0.2) (layer "B.Cu") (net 5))
 (segment (start 65.07 53.5) (end 63.42 51.85) (width 0.2) (layer "B.Cu") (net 5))
 (segment (start 84 52.0005) (end 85.0045 53.005) (width 0.2) (layer "B.Cu") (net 5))
 (segment (start 84 52) (end 84 48.5) (width 0.2) (layer "B.Cu") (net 5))
 (segment (start 84 48.5) (end 83.5 48) (width 0.2) (layer "B.Cu") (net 5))
 (segment (start 36 50.73) (end 35.8 50.53) (width 0.2) (layer "B.Cu") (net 5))
 (segment (start 52 50) (end 57.5 50) (width 0.2) (layer "B.Cu") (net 5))
 (segment (start 74.5 48) (end 74.03 48) (width 0.2) (layer "B.Cu") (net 5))
 (segment (start 78.5 53.5) (end 82 50) (width 0.2) (layer "B.Cu") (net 5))
 (segment (start 68.285 53.5) (end 65.07 53.5) (width 0.2) (layer "B.Cu") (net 5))
 (segment (start 70 56.5) (end 70 55) (width 0.2) (layer "B.Cu") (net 5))
 (segment (start 74.03 48) (end 71.88 50.15) (width 0.2) (layer "B.Cu") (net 5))
 (segment (start 41 56.25) (end 39.25 58) (width 0.2) (layer "B.Cu") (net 5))
 (segment (start 82 50) (end 82 49.5) (width 0.2) (layer "B.Cu") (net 5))
 (segment (start 82 49.5) (end 83.5 48) (width 0.2) (layer "B.Cu") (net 5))
 (segment (start 31.5 53) (end 33.0045 53) (width 0.2) (layer "B.Cu") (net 5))
 (segment (start 41 53.5) (end 41 56.25) (width 0.2) (layer "B.Cu") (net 5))
 (segment (start 84 52) (end 84 52.0005) (width 0.2) (layer "B.Cu") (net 5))
 (segment (start 69 57.5) (end 67.58 57.5) (width 0.2) (layer "B.Cu") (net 5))
 (segment (start 70 56.5) (end 69 57.5) (width 0.2) (layer "B.Cu") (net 5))
 (segment (start 32.405 55.405) (end 34.5 57.5) (width 0.2) (layer "F.Cu") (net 8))
 (segment (start 32.405 51.195) (end 32.405 55.405) (width 0.2) (layer "F.Cu") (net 8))
 (segment (start 33.1 50.5) (end 32.405 51.195) (width 0.2) (layer "F.Cu") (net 8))
 (segment (start 34.51 49.09) (end 33.1 50.5) (width 0.2) (layer "F.Cu") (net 8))
 (segment (start 34.51 48.5) (end 34.51 49.09) (width 0.2) (layer "F.Cu") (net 8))
 (segment (start 34.5 57.5) (end 52.34 57.5) (width 0.2) (layer "F.Cu") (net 8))
 (segment (start 49.1 51.715) (end 50.205 52.82) (width 0.2) (layer "F.Cu") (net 6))
 (segment (start 50.51 49.09) (end 50.51 48.5) (width 0.2) (layer "F.Cu") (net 6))
 (segment (start 50.205 55.338571) (end 51.241429 56.375) (width 0.2) (layer "F.Cu") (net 6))
 (segment (start 49.1 50.5) (end 50.51 49.09) (width 0.2) (layer "F.Cu") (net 6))
 (segment (start 50.205 52.82) (end 50.205 55.338571) (width 0.2) (layer "F.Cu") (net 6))
 (segment (start 51.241429 56.375) (end 53.755 56.375) (width 0.2) (layer "F.Cu") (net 6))
 (segment (start 49.1 50.5) (end 49.1 51.715) (width 0.2) (layer "F.Cu") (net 6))
 (segment (start 53.755 56.375) (end 54.88 57.5) (width 0.2) (layer "F.Cu") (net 6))
 (segment (start 64.01 49) (end 65.275 50.265) (width 0.2) (layer "F.Cu") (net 4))
 (segment (start 58.92 56) (end 57.42 57.5) (width 0.2) (layer "F.Cu") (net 4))
 (segment (start 62.1 49) (end 64.01 49) (width 0.2) (layer "F.Cu") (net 4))
 (segment (start 61.364314 56) (end 58.92 56) (width 0.2) (layer "F.Cu") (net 4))
 (segment (start 65.275 52.089314) (end 61.364314 56) (width 0.2) (layer "F.Cu") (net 4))
 (segment (start 65.275 50.265) (end 65.275 52.089314) (width 0.2) (layer "F.Cu") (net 4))
 (segment (start 62 49.1) (end 62.1 49) (width 0.2) (layer "F.Cu") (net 4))
 (segment (start 67.43 50.5) (end 60.43 57.5) (width 0.2) (layer "F.Cu") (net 9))
 (segment (start 60.43 57.5) (end 59.96 57.5) (width 0.2) (layer "F.Cu") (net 9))
 (segment (start 68.475 49.875) (end 69.1 50.5) (width 0.2) (layer "F.Cu") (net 9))
 (segment (start 69.735 47.725) (end 68.767893 47.725) (width 0.2) (layer "F.Cu") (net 9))
 (segment (start 69.1 50.5) (end 67.43 50.5) (width 0.2) (layer "F.Cu") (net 9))
 (segment (start 68.767893 47.725) (end 68.475 48.017893) (width 0.2) (layer "F.Cu") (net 9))
 (segment (start 70.51 48.5) (end 69.735 47.725) (width 0.2) (layer "F.Cu") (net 9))
 (segment (start 68.475 48.017893) (end 68.475 49.875) (width 0.2) (layer "F.Cu") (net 9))
 (segment (start 63.625 58.625) (end 62.5 57.5) (width 0.2) (layer "F.Cu") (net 10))
 (segment (start 86.51 48.5) (end 86.51 49.09) (width 0.2) (layer "F.Cu") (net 10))
 (segment (start 84.405 54.595) (end 80.375 58.625) (width 0.2) (layer "F.Cu") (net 10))
 (segment (start 86.51 49.09) (end 85.1 50.5) (width 0.2) (layer "F.Cu") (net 10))
 (segment (start 80.375 58.625) (end 63.625 58.625) (width 0.2) (layer "F.Cu") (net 10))
 (segment (start 85.1 50.5) (end 84.405 51.195) (width 0.2) (layer "F.Cu") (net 10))
 (segment (start 84.405 51.195) (end 84.405 54.595) (width 0.2) (layer "F.Cu") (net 10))
 (segment (start 37 50.175) (end 37 50.565) (width 0.2) (layer "F.Cu") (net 7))
 (segment (start 37 50.565) (end 34.9 52.665) (width 0.2) (layer "F.Cu") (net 7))
 (segment (start 34.9 52.665) (end 34.9 54.5) (width 0.2) (layer "F.Cu") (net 7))
 (segment (start 50.9 52.45) (end 50.9 54.5) (width 0.2) (layer "F.Cu") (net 11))
 (segment (start 53 50.35) (end 50.9 52.45) (width 0.2) (layer "F.Cu") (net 11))
 (segment (start 62.325 53.675) (end 62.325 53) (width 0.2) (layer "F.Cu") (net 3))
 (segment (start 58 50.9) (end 58 52) (width 0.2) (layer "F.Cu") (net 3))
 (segment (start 58 52) (end 58.5 52.5) (width 0.2) (layer "F.Cu") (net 3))
 (segment (start 62 54) (end 62.325 53.675) (width 0.2) (layer "F.Cu") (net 3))
 (via (at 62 54) (size 0.6) (drill 0.3) (layers "F.Cu" "B.Cu") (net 3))
 (via (at 58.5 52.5) (size 0.6) (drill 0.3) (layers "F.Cu" "B.Cu") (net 3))
 (segment (start 60 54) (end 62 54) (width 0.2) (layer "B.Cu") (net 3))
 (segment (start 60 54) (end 58.5 52.5) (width 0.2) (layer "B.Cu") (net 3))
 (segment (start 72.225 50.95) (end 73 50.175) (width 0.2) (layer "F.Cu") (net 12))
 (segment (start 70.9 54.5) (end 72.225 53.175) (width 0.2) (layer "F.Cu") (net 12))
 (segment (start 72.225 53.175) (end 72.225 50.95) (width 0.2) (layer "F.Cu") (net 12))
 (segment (start 86.9 53.925) (end 89 51.825) (width 0.2) (layer "F.Cu") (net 2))
 (segment (start 86.9 54.5) (end 86.9 53.925) (width 0.2) (layer "F.Cu") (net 2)))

